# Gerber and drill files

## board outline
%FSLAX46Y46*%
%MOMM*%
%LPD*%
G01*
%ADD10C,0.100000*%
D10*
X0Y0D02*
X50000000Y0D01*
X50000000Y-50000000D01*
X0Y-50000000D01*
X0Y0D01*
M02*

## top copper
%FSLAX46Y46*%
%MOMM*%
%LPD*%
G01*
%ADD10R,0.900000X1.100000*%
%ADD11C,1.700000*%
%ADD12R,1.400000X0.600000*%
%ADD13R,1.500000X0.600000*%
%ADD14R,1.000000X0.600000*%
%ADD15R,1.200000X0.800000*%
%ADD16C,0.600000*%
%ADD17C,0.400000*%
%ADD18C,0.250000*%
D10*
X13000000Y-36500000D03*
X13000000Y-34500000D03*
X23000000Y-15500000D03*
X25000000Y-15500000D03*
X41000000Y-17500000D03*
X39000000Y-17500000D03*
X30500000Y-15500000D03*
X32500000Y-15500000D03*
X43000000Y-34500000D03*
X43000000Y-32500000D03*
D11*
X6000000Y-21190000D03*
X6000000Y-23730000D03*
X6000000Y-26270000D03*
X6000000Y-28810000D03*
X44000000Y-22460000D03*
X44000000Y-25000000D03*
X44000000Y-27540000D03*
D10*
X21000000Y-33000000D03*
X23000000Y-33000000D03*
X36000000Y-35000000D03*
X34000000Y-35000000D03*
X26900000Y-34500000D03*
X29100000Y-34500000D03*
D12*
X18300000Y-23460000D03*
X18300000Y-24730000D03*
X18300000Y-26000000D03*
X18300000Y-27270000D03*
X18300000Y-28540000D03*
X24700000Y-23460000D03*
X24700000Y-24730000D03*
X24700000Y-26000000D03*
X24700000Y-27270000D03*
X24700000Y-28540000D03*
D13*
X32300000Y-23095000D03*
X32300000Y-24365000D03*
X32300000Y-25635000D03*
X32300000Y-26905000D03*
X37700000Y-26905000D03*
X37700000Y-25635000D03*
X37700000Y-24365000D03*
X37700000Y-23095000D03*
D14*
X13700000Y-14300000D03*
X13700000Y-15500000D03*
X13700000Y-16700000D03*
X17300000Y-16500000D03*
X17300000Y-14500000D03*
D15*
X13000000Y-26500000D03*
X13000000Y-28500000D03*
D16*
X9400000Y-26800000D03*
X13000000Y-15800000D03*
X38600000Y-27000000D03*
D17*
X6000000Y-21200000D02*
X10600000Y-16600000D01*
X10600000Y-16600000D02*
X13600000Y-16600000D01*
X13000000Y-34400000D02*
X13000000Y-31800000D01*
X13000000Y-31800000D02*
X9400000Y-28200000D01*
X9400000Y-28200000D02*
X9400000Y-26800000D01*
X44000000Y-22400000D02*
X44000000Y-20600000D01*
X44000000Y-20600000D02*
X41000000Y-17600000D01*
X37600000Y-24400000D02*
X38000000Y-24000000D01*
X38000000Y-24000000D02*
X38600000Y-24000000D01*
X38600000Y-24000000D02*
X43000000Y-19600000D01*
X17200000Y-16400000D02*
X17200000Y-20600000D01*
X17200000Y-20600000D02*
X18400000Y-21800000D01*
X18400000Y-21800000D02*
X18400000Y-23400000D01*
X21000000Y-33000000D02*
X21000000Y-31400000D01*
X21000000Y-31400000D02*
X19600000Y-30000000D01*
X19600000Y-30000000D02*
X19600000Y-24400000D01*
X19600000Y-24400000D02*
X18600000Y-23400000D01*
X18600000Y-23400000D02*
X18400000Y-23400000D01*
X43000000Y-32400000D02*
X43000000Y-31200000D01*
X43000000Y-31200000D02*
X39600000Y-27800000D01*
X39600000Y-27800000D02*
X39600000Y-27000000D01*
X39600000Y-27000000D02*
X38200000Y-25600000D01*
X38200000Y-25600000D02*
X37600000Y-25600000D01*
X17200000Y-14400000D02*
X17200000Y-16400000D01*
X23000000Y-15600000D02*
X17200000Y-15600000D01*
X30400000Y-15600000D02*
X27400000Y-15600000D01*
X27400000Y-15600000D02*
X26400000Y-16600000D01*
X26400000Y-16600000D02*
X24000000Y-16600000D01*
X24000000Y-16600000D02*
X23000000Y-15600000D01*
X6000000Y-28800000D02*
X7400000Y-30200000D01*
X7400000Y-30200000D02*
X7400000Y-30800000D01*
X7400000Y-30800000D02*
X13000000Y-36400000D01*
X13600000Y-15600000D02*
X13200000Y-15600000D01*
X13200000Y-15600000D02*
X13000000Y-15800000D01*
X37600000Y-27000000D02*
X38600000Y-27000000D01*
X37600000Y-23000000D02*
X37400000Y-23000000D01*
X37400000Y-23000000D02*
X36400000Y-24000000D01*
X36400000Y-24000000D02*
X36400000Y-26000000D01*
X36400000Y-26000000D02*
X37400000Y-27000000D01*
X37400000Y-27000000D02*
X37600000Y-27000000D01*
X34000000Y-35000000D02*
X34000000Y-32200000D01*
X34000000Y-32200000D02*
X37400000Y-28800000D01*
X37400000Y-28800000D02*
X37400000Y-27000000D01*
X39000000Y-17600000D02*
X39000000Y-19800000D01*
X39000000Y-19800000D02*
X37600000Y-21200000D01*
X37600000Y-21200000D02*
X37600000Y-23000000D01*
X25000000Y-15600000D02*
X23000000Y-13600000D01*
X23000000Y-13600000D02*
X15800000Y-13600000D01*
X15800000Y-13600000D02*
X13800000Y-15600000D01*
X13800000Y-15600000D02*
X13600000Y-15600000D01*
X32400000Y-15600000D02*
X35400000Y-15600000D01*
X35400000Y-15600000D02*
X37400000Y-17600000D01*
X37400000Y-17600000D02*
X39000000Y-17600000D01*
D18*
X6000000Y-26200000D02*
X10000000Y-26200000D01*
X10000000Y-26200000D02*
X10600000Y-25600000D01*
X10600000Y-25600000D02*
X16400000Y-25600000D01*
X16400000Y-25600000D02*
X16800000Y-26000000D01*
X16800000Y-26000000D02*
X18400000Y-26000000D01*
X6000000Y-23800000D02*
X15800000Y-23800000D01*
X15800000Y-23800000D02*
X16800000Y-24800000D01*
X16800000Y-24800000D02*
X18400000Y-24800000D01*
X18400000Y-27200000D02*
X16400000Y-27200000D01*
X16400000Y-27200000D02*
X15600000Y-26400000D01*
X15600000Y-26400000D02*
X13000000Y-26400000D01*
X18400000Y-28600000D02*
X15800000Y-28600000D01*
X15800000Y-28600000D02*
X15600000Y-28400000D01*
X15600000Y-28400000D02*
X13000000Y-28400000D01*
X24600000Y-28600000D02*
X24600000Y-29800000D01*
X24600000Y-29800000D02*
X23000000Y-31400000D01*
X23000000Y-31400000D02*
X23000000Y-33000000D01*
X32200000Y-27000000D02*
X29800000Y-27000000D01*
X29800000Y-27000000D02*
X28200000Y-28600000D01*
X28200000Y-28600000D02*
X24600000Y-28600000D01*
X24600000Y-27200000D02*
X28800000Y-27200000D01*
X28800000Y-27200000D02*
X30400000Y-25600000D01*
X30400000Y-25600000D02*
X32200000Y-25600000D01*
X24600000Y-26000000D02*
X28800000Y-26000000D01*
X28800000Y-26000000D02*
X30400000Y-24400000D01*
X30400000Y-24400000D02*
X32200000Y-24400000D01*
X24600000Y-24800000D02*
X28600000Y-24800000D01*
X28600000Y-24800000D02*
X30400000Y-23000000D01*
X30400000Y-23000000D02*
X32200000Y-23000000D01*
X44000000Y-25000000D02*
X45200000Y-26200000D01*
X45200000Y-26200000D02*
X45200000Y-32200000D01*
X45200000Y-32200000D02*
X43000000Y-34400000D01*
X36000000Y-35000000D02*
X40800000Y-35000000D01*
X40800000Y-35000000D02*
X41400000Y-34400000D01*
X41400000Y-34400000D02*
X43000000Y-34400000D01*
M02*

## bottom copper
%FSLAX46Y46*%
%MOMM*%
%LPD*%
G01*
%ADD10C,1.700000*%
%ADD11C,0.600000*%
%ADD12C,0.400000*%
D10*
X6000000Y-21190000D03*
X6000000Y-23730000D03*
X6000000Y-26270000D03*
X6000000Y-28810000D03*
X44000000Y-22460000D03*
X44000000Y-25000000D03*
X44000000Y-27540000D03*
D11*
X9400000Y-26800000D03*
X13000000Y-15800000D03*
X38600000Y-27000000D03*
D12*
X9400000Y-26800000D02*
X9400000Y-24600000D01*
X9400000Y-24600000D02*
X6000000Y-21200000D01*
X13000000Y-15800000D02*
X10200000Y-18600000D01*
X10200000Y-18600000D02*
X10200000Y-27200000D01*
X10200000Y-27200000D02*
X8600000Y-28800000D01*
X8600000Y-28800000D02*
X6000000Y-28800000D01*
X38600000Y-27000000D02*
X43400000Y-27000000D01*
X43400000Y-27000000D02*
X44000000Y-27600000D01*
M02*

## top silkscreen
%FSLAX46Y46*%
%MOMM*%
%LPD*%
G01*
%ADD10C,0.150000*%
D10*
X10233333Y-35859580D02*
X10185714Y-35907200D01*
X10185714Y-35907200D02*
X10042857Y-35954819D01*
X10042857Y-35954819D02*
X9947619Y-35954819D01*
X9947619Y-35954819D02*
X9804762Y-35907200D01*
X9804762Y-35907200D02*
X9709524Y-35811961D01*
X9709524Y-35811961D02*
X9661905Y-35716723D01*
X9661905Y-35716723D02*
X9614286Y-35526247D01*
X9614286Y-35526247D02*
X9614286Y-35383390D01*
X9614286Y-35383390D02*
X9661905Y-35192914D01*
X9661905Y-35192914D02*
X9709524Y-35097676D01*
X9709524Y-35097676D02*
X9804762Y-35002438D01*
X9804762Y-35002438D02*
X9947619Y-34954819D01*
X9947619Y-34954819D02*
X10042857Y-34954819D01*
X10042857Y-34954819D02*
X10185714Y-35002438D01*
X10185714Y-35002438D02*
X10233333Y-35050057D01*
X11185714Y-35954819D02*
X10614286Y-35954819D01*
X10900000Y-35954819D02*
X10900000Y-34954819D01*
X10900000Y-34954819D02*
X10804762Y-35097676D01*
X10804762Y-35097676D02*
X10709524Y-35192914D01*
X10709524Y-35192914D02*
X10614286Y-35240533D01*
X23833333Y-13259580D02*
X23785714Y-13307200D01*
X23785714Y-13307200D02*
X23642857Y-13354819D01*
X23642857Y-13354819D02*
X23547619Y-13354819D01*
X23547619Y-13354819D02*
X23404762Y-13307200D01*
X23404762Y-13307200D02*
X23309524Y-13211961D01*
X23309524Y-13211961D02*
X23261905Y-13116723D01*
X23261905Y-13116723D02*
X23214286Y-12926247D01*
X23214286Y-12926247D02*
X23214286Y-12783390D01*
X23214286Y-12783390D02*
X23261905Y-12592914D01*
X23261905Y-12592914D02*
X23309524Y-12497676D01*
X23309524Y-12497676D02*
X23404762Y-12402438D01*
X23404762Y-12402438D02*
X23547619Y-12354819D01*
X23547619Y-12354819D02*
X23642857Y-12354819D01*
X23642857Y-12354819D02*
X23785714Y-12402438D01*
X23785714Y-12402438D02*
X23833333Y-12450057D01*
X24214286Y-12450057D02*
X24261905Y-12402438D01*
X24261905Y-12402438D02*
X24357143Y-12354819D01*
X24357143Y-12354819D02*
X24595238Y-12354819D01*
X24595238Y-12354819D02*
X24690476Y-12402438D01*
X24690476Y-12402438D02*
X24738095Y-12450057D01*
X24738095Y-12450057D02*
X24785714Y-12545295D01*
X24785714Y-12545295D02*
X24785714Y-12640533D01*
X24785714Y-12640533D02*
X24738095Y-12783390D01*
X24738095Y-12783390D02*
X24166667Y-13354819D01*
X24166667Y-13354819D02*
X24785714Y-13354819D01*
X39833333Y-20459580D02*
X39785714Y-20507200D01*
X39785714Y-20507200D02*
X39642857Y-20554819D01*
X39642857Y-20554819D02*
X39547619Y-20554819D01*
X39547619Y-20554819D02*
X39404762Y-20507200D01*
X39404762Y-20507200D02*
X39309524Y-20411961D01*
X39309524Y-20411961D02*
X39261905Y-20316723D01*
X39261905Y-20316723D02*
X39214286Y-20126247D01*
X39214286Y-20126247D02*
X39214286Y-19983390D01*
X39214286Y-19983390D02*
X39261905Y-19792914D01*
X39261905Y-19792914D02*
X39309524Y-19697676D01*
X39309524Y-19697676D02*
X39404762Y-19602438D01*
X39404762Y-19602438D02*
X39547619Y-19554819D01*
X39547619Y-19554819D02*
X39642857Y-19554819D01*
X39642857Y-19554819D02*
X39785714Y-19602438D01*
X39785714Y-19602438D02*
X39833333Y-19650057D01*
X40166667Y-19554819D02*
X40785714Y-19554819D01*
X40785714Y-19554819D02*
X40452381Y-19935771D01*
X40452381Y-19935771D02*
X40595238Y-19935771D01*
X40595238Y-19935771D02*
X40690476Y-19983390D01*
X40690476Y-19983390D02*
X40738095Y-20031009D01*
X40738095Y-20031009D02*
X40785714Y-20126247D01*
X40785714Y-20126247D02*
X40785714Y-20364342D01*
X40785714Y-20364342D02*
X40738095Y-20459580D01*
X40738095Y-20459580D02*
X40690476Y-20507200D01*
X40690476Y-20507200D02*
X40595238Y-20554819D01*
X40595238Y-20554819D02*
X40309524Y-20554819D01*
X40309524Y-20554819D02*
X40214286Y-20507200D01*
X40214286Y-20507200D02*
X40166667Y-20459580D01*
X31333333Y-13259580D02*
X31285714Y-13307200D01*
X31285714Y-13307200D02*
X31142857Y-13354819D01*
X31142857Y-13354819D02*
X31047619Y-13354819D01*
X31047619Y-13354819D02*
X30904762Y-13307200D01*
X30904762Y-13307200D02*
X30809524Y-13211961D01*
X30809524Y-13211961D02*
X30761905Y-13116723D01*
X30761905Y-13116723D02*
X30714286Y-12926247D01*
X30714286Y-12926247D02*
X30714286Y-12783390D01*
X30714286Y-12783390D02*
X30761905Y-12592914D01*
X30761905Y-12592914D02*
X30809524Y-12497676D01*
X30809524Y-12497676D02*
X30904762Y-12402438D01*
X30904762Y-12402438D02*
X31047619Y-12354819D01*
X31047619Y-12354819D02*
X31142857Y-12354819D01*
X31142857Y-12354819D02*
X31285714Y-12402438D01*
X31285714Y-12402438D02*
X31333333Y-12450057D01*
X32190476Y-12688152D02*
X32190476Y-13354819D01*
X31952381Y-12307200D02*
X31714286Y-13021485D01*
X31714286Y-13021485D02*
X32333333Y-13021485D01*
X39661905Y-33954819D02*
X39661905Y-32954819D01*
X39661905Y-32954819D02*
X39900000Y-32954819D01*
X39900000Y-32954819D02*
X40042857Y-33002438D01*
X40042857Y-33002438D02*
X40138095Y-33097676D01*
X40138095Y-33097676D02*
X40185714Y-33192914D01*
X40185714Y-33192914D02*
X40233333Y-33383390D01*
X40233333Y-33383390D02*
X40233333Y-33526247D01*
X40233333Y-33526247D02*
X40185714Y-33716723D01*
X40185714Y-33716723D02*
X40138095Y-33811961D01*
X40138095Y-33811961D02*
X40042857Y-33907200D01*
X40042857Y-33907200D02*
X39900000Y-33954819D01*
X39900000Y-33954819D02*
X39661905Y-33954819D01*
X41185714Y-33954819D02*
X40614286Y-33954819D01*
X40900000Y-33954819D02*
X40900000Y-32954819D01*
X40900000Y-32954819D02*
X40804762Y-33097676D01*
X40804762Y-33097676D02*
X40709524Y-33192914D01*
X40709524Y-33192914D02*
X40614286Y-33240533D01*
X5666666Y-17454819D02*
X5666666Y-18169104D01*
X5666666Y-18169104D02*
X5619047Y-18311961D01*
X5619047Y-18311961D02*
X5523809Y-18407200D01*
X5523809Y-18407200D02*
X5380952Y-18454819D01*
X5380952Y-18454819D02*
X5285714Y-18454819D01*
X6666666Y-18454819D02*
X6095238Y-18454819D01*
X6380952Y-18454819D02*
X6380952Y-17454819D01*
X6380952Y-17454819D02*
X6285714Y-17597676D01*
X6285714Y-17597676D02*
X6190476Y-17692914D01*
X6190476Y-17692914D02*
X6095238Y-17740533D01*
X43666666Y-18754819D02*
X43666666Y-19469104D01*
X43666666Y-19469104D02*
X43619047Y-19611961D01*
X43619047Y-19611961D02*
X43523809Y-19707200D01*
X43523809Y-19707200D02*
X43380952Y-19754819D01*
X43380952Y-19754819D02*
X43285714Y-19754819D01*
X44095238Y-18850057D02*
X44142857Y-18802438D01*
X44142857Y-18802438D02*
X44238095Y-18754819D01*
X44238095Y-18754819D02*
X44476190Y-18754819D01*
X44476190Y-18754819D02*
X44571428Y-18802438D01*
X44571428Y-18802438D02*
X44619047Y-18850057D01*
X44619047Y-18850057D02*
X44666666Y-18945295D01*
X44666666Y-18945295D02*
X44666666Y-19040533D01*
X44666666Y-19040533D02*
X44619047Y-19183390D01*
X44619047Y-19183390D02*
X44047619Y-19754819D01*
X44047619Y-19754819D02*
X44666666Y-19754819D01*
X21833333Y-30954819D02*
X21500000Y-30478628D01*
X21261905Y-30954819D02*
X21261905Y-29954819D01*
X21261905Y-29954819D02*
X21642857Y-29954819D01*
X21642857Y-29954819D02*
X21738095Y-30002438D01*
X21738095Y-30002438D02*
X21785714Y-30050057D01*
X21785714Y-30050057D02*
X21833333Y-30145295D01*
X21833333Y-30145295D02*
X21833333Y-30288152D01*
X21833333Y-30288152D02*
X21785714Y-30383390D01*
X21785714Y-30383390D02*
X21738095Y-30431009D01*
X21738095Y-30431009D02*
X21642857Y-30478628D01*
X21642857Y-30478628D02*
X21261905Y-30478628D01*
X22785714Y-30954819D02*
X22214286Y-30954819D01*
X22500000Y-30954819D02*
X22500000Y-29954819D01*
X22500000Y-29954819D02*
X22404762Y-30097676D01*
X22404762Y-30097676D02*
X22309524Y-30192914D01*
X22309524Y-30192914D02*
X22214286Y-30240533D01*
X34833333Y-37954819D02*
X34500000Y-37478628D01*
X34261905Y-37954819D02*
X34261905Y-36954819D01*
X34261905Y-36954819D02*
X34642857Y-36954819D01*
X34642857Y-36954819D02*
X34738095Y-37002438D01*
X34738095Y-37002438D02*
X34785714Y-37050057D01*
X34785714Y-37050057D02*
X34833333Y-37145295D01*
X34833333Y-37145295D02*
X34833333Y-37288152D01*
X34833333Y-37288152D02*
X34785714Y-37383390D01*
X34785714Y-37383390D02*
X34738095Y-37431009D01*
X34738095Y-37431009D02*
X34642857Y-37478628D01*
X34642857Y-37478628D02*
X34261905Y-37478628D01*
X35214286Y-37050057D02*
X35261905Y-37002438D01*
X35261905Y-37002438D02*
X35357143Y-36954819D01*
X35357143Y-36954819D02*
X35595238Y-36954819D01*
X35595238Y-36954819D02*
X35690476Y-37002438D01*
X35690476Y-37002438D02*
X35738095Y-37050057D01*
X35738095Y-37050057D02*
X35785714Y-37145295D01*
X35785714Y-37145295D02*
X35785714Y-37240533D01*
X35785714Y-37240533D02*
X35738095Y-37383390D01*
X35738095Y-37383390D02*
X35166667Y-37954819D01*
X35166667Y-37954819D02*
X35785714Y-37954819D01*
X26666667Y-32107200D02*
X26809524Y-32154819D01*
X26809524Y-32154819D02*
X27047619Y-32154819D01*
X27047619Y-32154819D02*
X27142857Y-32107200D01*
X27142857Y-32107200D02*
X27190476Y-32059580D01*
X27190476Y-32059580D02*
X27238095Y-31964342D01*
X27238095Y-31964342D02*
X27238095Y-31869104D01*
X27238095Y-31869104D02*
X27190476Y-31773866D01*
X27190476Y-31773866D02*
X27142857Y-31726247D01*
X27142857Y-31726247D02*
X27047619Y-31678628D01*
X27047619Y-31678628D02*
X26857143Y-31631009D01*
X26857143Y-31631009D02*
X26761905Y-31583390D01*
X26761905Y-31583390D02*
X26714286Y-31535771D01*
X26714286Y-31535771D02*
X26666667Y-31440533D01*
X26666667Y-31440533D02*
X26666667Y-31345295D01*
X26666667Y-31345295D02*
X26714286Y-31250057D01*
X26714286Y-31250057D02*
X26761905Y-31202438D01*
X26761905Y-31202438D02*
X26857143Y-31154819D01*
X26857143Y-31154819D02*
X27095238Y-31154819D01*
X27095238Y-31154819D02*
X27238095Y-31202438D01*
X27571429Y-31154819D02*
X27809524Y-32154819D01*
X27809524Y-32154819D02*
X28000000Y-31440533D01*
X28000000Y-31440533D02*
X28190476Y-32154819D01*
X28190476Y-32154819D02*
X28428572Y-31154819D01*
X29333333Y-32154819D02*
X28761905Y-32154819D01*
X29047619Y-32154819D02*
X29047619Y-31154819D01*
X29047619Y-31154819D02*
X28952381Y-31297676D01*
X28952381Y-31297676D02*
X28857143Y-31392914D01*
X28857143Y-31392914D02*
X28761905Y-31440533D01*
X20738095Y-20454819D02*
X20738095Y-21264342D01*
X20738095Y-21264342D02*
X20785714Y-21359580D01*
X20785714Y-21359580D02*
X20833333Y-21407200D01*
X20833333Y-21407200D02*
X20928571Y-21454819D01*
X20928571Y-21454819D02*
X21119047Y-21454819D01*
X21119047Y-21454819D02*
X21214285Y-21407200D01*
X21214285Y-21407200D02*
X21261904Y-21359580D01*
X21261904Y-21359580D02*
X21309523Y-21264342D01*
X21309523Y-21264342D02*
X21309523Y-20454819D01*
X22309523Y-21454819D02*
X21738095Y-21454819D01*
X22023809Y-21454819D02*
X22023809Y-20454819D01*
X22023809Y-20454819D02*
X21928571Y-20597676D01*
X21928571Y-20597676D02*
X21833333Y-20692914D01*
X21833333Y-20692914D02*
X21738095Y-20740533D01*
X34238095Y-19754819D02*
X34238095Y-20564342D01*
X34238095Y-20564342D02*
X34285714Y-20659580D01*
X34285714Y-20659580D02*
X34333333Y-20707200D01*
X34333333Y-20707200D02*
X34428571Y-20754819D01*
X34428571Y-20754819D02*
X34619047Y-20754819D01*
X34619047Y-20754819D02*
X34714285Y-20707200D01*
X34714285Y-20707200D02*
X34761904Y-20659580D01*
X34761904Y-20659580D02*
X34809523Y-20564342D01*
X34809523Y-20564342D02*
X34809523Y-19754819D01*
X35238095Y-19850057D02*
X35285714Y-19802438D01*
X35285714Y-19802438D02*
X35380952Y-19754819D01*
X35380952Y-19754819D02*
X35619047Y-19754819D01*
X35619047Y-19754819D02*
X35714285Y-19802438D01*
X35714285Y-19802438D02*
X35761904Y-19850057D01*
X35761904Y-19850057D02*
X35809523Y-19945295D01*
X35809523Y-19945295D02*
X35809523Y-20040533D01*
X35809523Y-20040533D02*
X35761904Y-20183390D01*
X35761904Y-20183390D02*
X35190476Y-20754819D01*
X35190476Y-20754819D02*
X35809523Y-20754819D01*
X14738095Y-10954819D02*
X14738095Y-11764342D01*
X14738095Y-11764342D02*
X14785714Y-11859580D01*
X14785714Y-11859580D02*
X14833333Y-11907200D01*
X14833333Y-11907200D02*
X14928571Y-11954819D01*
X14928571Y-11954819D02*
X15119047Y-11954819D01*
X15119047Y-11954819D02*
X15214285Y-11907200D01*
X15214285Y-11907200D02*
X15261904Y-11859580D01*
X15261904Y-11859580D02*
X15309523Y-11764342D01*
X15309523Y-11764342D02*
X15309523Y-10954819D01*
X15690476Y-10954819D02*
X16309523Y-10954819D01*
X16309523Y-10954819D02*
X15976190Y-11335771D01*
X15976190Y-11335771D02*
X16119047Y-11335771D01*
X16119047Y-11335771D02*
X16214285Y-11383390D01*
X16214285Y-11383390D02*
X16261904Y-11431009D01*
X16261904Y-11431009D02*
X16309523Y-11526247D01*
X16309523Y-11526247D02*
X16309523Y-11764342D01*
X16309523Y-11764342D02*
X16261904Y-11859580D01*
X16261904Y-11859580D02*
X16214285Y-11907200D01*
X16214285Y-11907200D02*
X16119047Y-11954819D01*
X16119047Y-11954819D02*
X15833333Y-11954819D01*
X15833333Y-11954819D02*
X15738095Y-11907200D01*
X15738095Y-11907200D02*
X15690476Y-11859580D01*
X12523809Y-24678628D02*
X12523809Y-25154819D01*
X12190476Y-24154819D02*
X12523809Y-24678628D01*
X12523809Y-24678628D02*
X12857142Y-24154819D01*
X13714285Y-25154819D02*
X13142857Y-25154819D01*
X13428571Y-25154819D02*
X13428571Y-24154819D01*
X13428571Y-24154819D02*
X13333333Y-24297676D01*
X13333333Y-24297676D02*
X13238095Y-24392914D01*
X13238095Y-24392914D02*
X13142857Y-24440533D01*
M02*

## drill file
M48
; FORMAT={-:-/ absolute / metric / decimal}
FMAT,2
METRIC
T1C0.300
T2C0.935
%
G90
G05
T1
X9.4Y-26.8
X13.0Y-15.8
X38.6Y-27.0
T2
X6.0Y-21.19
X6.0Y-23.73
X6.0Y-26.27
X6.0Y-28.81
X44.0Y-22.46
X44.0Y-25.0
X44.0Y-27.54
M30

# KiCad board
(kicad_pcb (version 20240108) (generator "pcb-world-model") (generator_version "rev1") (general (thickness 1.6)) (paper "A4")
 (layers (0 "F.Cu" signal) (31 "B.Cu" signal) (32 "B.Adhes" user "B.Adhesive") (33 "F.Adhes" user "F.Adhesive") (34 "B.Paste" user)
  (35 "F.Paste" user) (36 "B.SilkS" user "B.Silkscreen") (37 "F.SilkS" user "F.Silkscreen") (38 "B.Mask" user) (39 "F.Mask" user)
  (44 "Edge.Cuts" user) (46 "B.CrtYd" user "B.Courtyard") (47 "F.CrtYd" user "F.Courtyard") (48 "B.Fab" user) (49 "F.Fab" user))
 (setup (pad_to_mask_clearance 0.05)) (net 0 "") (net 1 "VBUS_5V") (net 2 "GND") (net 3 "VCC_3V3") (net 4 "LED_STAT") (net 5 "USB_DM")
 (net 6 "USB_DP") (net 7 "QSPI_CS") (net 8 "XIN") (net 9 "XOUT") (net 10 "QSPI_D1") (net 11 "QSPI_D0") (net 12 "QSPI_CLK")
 (gr_rect (start 0.0 0.0) (end 50.0000 50.0000) (stroke (width 0.1) (type default)) (fill none) (layer "Edge.Cuts"))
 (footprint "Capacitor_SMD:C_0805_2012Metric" (layer "F.Cu") (at 13.0000 35.5000 90)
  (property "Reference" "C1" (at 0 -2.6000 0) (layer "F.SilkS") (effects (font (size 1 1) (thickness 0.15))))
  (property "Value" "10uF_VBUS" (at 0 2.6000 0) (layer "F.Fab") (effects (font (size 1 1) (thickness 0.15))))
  (pad "1" smd rect (at -1.0000 0.0000) (size 0.9000 1.1000) (layers "F.Cu" "F.Paste" "F.Mask") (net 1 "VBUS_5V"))
  (pad "2" smd rect (at 1.0000 0.0000) (size 0.9000 1.1000) (layers "F.Cu" "F.Paste" "F.Mask") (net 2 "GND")))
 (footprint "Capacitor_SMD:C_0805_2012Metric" (layer "F.Cu") (at 24.0000 15.5000 0)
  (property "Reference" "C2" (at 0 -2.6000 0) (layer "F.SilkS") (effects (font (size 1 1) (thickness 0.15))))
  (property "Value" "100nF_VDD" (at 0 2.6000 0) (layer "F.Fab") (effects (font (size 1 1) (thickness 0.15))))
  (pad "1" smd rect (at -1.0000 0.0000) (size 0.9000 1.1000) (layers "F.Cu" "F.Paste" "F.Mask") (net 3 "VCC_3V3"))
  (pad "2" smd rect (at 1.0000 0.0000) (size 0.9000 1.1000) (layers "F.Cu" "F.Paste" "F.Mask") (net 2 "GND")))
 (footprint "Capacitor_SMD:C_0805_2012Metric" (layer "F.Cu") (at 40.0000 17.5000 180)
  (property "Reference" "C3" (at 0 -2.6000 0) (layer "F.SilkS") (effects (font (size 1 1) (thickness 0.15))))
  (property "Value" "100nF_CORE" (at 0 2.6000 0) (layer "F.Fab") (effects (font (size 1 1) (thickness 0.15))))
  (pad "1" smd rect (at -1.0000 0.0000) (size 0.9000 1.1000) (layers "F.Cu" "F.Paste" "F.Mask") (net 3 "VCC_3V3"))
  (pad "2" smd rect (at 1.0000 0.0000) (size 0.9000 1.1000) (layers "F.Cu" "F.Paste" "F.Mask") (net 2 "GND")))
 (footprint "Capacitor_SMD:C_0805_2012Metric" (layer "F.Cu") (at 31.5000 15.5000 0)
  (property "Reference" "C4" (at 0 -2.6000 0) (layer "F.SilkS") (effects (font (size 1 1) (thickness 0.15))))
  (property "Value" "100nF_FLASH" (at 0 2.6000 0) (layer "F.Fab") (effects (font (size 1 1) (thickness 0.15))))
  (pad "1" smd rect (at -1.0000 0.0000) (size 0.9000 1.1000) (layers "F.Cu" "F.Paste" "F.Mask") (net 3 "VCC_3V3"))
  (pad "2" smd rect (at 1.0000 0.0000) (size 0.9000 1.1000) (layers "F.Cu" "F.Paste" "F.Mask") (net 2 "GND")))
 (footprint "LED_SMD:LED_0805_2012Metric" (layer "F.Cu") (at 43.0000 33.5000 90)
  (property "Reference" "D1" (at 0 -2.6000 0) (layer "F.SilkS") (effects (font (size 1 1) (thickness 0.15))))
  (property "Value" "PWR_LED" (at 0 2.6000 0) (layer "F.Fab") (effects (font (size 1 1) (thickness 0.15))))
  (pad "1" smd rect (at -1.0000 0.0000) (size 0.9000 1.1000) (layers "F.Cu" "F.Paste" "F.Mask") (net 3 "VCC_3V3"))
  (pad "2" smd rect (at 1.0000 0.0000) (size 0.9000 1.1000) (layers "F.Cu" "F.Paste" "F.Mask") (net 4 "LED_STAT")))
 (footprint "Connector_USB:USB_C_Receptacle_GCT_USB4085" (layer "F.Cu") (at 6.0000 25.0000 0) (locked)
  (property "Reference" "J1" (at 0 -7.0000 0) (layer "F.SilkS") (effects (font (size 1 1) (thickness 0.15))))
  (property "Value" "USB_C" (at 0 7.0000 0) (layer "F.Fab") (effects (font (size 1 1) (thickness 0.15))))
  (pad "1" thru_hole circle (at 0.0000 -3.8100) (size 1.7000 1.7000) (drill 0.9350) (layers "*.Cu" "*.Mask") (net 1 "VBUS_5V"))
  (pad "2" thru_hole circle (at 0.0000 -1.2700) (size 1.7000 1.7000) (drill 0.9350) (layers "*.Cu" "*.Mask") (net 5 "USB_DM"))
  (pad "3" thru_hole circle (at 0.0000 1.2700) (size 1.7000 1.7000) (drill 0.9350) (layers "*.Cu" "*.Mask") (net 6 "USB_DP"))
  (pad "4" thru_hole circle (at 0.0000 3.8100) (size 1.7000 1.7000) (drill 0.9350) (layers "*.Cu" "*.Mask") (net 2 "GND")))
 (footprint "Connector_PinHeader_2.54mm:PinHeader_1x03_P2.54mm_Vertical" (layer "F.Cu") (at 44.0000 25.0000 0) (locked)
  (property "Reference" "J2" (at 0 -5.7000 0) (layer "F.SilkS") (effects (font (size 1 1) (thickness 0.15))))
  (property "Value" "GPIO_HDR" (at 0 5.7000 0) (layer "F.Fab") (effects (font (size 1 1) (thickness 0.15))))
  (pad "1" thru_hole circle (at 0.0000 -2.5400) (size 1.7000 1.7000) (drill 0.9350) (layers "*.Cu" "*.Mask") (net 3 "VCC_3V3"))
  (pad "2" thru_hole circle (at 0.0000 0.0000) (size 1.7000 1.7000) (drill 0.9350) (layers "*.Cu" "*.Mask") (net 4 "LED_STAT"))
  (pad "3" thru_hole circle (at 0.0000 2.5400) (size 1.7000 1.7000) (drill 0.9350) (layers "*.Cu" "*.Mask") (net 2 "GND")))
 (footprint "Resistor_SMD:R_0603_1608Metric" (layer "F.Cu") (at 22.0000 33.0000 0)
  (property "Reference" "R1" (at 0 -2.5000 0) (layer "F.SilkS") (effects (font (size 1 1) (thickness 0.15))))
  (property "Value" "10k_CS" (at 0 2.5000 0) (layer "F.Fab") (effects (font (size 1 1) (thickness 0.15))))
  (pad "1" smd rect (at -1.0000 0.0000) (size 0.9000 1.1000) (layers "F.Cu" "F.Paste" "F.Mask") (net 3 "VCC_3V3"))
  (pad "2" smd rect (at 1.0000 0.0000) (size 0.9000 1.1000) (layers "F.Cu" "F.Paste" "F.Mask") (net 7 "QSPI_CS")))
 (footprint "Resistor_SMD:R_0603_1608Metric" (layer "F.Cu") (at 35.0000 35.0000 180)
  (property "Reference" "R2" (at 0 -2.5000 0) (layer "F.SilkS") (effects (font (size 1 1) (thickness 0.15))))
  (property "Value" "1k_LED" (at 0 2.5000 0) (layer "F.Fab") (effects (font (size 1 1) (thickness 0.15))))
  (pad "1" smd rect (at -1.0000 0.0000) (size 0.9000 1.1000) (layers "F.Cu" "F.Paste" "F.Mask") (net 4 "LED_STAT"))
  (pad "2" smd rect (at 1.0000 0.0000) (size 0.9000 1.1000) (layers "F.Cu" "F.Paste" "F.Mask") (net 2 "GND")))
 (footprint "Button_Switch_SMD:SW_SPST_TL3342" (layer "F.Cu") (at 28.0000 34.5000 0)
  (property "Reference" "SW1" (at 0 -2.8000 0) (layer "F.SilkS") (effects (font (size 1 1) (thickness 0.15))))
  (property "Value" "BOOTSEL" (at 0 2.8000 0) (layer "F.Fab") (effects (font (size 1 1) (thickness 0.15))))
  (pad "1" smd rect (at -1.1000 0.0000) (size 0.9000 1.1000) (layers "F.Cu" "F.Paste" "F.Mask") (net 7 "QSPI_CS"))
  (pad "2" smd rect (at 1.1000 0.0000) (size 0.9000 1.1000) (layers "F.Cu" "F.Paste" "F.Mask") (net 2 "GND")))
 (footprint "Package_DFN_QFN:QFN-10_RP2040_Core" (layer "F.Cu") (at 21.5000 26.0000 0)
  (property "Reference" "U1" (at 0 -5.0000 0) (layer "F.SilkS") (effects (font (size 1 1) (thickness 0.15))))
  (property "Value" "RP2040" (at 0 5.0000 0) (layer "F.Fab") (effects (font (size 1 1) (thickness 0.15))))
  (pad "1" smd rect (at -3.2000 -2.5400) (size 1.4000 0.6000) (layers "F.Cu" "F.Paste" "F.Mask") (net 3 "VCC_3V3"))
  (pad "2" smd rect (at -3.2000 -1.2700) (size 1.4000 0.6000) (layers "F.Cu" "F.Paste" "F.Mask") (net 5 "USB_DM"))
  (pad "3" smd rect (at -3.2000 0.0000) (size 1.4000 0.6000) (layers "F.Cu" "F.Paste" "F.Mask") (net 6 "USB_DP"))
  (pad "4" smd rect (at -3.2000 1.2700) (size 1.4000 0.6000) (layers "F.Cu" "F.Paste" "F.Mask") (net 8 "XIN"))
  (pad "5" smd rect (at -3.2000 2.5400) (size 1.4000 0.6000) (layers "F.Cu" "F.Paste" "F.Mask") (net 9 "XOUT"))
  (pad "6" smd rect (at 3.2000 -2.5400) (size 1.4000 0.6000) (layers "F.Cu" "F.Paste" "F.Mask") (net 4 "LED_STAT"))
  (pad "7" smd rect (at 3.2000 -1.2700) (size 1.4000 0.6000) (layers "F.Cu" "F.Paste" "F.Mask") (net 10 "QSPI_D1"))
  (pad "8" smd rect (at 3.2000 0.0000) (size 1.4000 0.6000) (layers "F.Cu" "F.Paste" "F.Mask") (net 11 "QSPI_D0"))
  (pad "9" smd rect (at 3.2000 1.2700) (size 1.4000 0.6000) (layers "F.Cu" "F.Paste" "F.Mask") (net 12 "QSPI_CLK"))
  (pad "10" smd rect (at 3.2000 2.5400) (size 1.4000 0.6000) (layers "F.Cu" "F.Paste" "F.Mask") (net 7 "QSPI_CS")))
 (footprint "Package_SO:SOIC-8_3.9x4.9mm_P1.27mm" (layer "F.Cu") (at 35.0000 25.0000 0)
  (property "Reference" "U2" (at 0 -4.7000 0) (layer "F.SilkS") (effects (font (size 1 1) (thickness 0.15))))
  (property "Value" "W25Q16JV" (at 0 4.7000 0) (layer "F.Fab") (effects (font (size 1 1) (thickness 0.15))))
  (pad "1" smd rect (at -2.7000 -1.9050) (size 1.5000 0.6000) (layers "F.Cu" "F.Paste" "F.Mask") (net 10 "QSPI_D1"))
  (pad "2" smd rect (at -2.7000 -0.6350) (size 1.5000 0.6000) (layers "F.Cu" "F.Paste" "F.Mask") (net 11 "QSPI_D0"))
  (pad "3" smd rect (at -2.7000 0.6350) (size 1.5000 0.6000) (layers "F.Cu" "F.Paste" "F.Mask") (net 12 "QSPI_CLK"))
  (pad "4" smd rect (at -2.7000 1.9050) (size 1.5000 0.6000) (layers "F.Cu" "F.Paste" "F.Mask") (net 7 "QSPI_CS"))
  (pad "5" smd rect (at 2.7000 1.9050) (size 1.5000 0.6000) (layers "F.Cu" "F.Paste" "F.Mask") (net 2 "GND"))
  (pad "6" smd rect (at 2.7000 0.6350) (size 1.5000 0.6000) (layers "F.Cu" "F.Paste" "F.Mask") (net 3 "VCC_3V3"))
  (pad "7" smd rect (at 2.7000 -0.6350) (size 1.5000 0.6000) (layers "F.Cu" "F.Paste" "F.Mask") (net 3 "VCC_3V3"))
  (pad "8" smd rect (at 2.7000 -1.9050) (size 1.5000 0.6000) (layers "F.Cu" "F.Paste" "F.Mask") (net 2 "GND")))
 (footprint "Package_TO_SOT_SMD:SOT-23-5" (layer "F.Cu") (at 15.5000 15.5000 0)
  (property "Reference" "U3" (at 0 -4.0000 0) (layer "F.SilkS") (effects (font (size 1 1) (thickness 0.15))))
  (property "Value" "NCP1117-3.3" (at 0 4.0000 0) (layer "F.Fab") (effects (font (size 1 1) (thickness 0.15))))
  (pad "1" smd rect (at -1.8000 -1.2000) (size 1.0000 0.6000) (layers "F.Cu" "F.Paste" "F.Mask") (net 1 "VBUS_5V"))
  (pad "2" smd rect (at -1.8000 0.0000) (size 1.0000 0.6000) (layers "F.Cu" "F.Paste" "F.Mask") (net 2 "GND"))
  (pad "3" smd rect (at -1.8000 1.2000) (size 1.0000 0.6000) (layers "F.Cu" "F.Paste" "F.Mask") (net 1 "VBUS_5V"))
  (pad "4" smd rect (at 1.8000 1.0000) (size 1.0000 0.6000) (layers "F.Cu" "F.Paste" "F.Mask") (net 3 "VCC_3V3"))
  (pad "5" smd rect (at 1.8000 -1.0000) (size 1.0000 0.6000) (layers "F.Cu" "F.Paste" "F.Mask") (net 3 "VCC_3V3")))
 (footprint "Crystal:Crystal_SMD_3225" (layer "F.Cu") (at 13.0000 27.5000 0)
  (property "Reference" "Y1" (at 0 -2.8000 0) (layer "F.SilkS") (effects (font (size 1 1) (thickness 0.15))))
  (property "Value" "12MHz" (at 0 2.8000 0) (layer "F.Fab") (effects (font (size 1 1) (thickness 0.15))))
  (pad "1" smd rect (at 0.0000 -1.0000) (size 1.2000 0.8000) (layers "F.Cu" "F.Paste" "F.Mask") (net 8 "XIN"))
  (pad "2" smd rect (at 0.0000 1.0000) (size 1.2000 0.8000) (layers "F.Cu" "F.Paste" "F.Mask") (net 9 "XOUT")))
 (segment (start 6.0000 21.2000) (end 10.6000 16.6000) (width 0.4000) (layer "F.Cu") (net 1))
 (segment (start 10.6000 16.6000) (end 13.6000 16.6000) (width 0.4000) (layer "F.Cu") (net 1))
 (segment (start 13.0000 34.4000) (end 13.0000 31.8000) (width 0.4000) (layer "F.Cu") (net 1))
 (segment (start 13.0000 31.8000) (end 9.4000 28.2000) (width 0.4000) (layer "F.Cu") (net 1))
 (segment (start 9.4000 28.2000) (end 9.4000 26.8000) (width 0.4000) (layer "F.Cu") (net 1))
 (segment (start 9.4000 26.8000) (end 9.4000 24.6000) (width 0.4000) (layer "B.Cu") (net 1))
 (segment (start 9.4000 24.6000) (end 6.0000 21.2000) (width 0.4000) (layer "B.Cu") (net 1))
 (segment (start 44.0000 22.4000) (end 44.0000 20.6000) (width 0.4000) (layer "F.Cu") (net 3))
 (segment (start 44.0000 20.6000) (end 41.0000 17.6000) (width 0.4000) (layer "F.Cu") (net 3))
 (segment (start 37.6000 24.4000) (end 38.0000 24.0000) (width 0.4000) (layer "F.Cu") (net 3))
 (segment (start 38.0000 24.0000) (end 38.6000 24.0000) (width 0.4000) (layer "F.Cu") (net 3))
 (segment (start 38.6000 24.0000) (end 43.0000 19.6000) (width 0.4000) (layer "F.Cu") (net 3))
 (segment (start 17.2000 16.4000) (end 17.2000 20.6000) (width 0.4000) (layer "F.Cu") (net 3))
 (segment (start 17.2000 20.6000) (end 18.4000 21.8000) (width 0.4000) (layer "F.Cu") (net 3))
 (segment (start 18.4000 21.8000) (end 18.4000 23.4000) (width 0.4000) (layer "F.Cu") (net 3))
 (segment (start 21.0000 33.0000) (end 21.0000 31.4000) (width 0.4000) (layer "F.Cu") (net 3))
 (segment (start 21.0000 31.4000) (end 19.6000 30.0000) (width 0.4000) (layer "F.Cu") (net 3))
 (segment (start 19.6000 30.0000) (end 19.6000 24.4000) (width 0.4000) (layer "F.Cu") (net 3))
 (segment (start 19.6000 24.4000) (end 18.6000 23.4000) (width 0.4000) (layer "F.Cu") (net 3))
 (segment (start 18.6000 23.4000) (end 18.4000 23.4000) (width 0.4000) (layer "F.Cu") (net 3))
 (segment (start 43.0000 32.4000) (end 43.0000 31.2000) (width 0.4000) (layer "F.Cu") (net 3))
 (segment (start 43.0000 31.2000) (end 39.6000 27.8000) (width 0.4000) (layer "F.Cu") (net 3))
 (segment (start 39.6000 27.8000) (end 39.6000 27.0000) (width 0.4000) (layer "F.Cu") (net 3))
 (segment (start 39.6000 27.0000) (end 38.2000 25.6000) (width 0.4000) (layer "F.Cu") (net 3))
 (segment (start 38.2000 25.6000) (end 37.6000 25.6000) (width 0.4000) (layer "F.Cu") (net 3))
 (segment (start 17.2000 14.4000) (end 17.2000 16.4000) (width 0.4000) (layer "F.Cu") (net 3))
 (segment (start 23.0000 15.6000) (end 17.2000 15.6000) (width 0.4000) (layer "F.Cu") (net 3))
 (segment (start 30.4000 15.6000) (end 27.4000 15.6000) (width 0.4000) (layer "F.Cu") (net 3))
 (segment (start 27.4000 15.6000) (end 26.4000 16.6000) (width 0.4000) (layer "F.Cu") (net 3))
 (segment (start 26.4000 16.6000) (end 24.0000 16.6000) (width 0.4000) (layer "F.Cu") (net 3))
 (segment (start 24.0000 16.6000) (end 23.0000 15.6000) (width 0.4000) (layer "F.Cu") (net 3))
 (segment (start 6.0000 28.8000) (end 7.4000 30.2000) (width 0.4000) (layer "F.Cu") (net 2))
 (segment (start 7.4000 30.2000) (end 7.4000 30.8000) (width 0.4000) (layer "F.Cu") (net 2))
 (segment (start 7.4000 30.8000) (end 13.0000 36.4000) (width 0.4000) (layer "F.Cu") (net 2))
 (segment (start 13.6000 15.6000) (end 13.2000 15.6000) (width 0.4000) (layer "F.Cu") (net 2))
 (segment (start 13.2000 15.6000) (end 13.0000 15.8000) (width 0.4000) (layer "F.Cu") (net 2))
 (segment (start 13.0000 15.8000) (end 10.2000 18.6000) (width 0.4000) (layer "B.Cu") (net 2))
 (segment (start 10.2000 18.6000) (end 10.2000 27.2000) (width 0.4000) (layer "B.Cu") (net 2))
 (segment (start 10.2000 27.2000) (end 8.6000 28.8000) (width 0.4000) (layer "B.Cu") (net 2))
 (segment (start 8.6000 28.8000) (end 6.0000 28.8000) (width 0.4000) (layer "B.Cu") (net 2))
 (segment (start 37.6000 27.0000) (end 38.6000 27.0000) (width 0.4000) (layer "F.Cu") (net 2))
 (segment (start 38.6000 27.0000) (end 43.4000 27.0000) (width 0.4000) (layer "B.Cu") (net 2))
 (segment (start 43.4000 27.0000) (end 44.0000 27.6000) (width 0.4000) (layer "B.Cu") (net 2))
 (segment (start 37.6000 23.0000) (end 37.4000 23.0000) (width 0.4000) (layer "F.Cu") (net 2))
 (segment (start 37.4000 23.0000) (end 36.4000 24.0000) (width 0.4000) (layer "F.Cu") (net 2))
 (segment (start 36.4000 24.0000) (end 36.4000 26.0000) (width 0.4000) (layer "F.Cu") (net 2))
 (segment (start 36.4000 26.0000) (end 37.4000 27.0000) (width 0.4000) (layer "F.Cu") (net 2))
 (segment (start 37.4000 27.0000) (end 37.6000 27.0000) (width 0.4000) (layer "F.Cu") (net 2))
 (segment (start 34.0000 35.0000) (end 34.0000 32.2000) (width 0.4000) (layer "F.Cu") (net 2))
 (segment (start 34.0000 32.2000) (end 37.4000 28.8000) (width 0.4000) (layer "F.Cu") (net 2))
 (segment (start 37.4000 28.8000) (end 37.4000 27.0000) (width 0.4000) (layer "F.Cu") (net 2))
 (segment (start 39.0000 17.6000) (end 39.0000 19.8000) (width 0.4000) (layer "F.Cu") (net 2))
 (segment (start 39.0000 19.8000) (end 37.6000 21.2000) (width 0.4000) (layer "F.Cu") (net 2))
 (segment (start 37.6000 21.2000) (end 37.6000 23.0000) (width 0.4000) (layer "F.Cu") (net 2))
 (segment (start 25.0000 15.6000) (end 23.0000 13.6000) (width 0.4000) (layer "F.Cu") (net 2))
 (segment (start 23.0000 13.6000) (end 15.8000 13.6000) (width 0.4000) (layer "F.Cu") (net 2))
 (segment (start 15.8000 13.6000) (end 13.8000 15.6000) (width 0.4000) (layer "F.Cu") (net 2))
 (segment (start 13.8000 15.6000) (end 13.6000 15.6000) (width 0.4000) (layer "F.Cu") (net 2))
 (segment (start 32.4000 15.6000) (end 35.4000 15.6000) (width 0.4000) (layer "F.Cu") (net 2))
 (segment (start 35.4000 15.6000) (end 37.4000 17.6000) (width 0.4000) (layer "F.Cu") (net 2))
 (segment (start 37.4000 17.6000) (end 39.0000 17.6000) (width 0.4000) (layer "F.Cu") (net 2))
 (segment (start 6.0000 26.2000) (end 10.0000 26.2000) (width 0.2500) (layer "F.Cu") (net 6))
 (segment (start 10.0000 26.2000) (end 10.6000 25.6000) (width 0.2500) (layer "F.Cu") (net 6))
 (segment (start 10.6000 25.6000) (end 16.4000 25.6000) (width 0.2500) (layer "F.Cu") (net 6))
 (segment (start 16.4000 25.6000) (end 16.8000 26.0000) (width 0.2500) (layer "F.Cu") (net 6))
 (segment (start 16.8000 26.0000) (end 18.4000 26.0000) (width 0.2500) (layer "F.Cu") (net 6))
 (segment (start 6.0000 23.8000) (end 15.8000 23.8000) (width 0.2500) (layer "F.Cu") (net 5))
 (segment (start 15.8000 23.8000) (end 16.8000 24.8000) (width 0.2500) (layer "F.Cu") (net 5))
 (segment (start 16.8000 24.8000) (end 18.4000 24.8000) (width 0.2500) (layer "F.Cu") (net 5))
 (segment (start 18.4000 27.2000) (end 16.4000 27.2000) (width 0.2500) (layer "F.Cu") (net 8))
 (segment (start 16.4000 27.2000) (end 15.6000 26.4000) (width 0.2500) (layer "F.Cu") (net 8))
 (segment (start 15.6000 26.4000) (end 13.0000 26.4000) (width 0.2500) (layer "F.Cu") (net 8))
 (segment (start 18.4000 28.6000) (end 15.8000 28.6000) (width 0.2500) (layer "F.Cu") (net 9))
 (segment (start 15.8000 28.6000) (end 15.6000 28.4000) (width 0.2500) (layer "F.Cu") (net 9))
 (segment (start 15.6000 28.4000) (end 13.0000 28.4000) (width 0.2500) (layer "F.Cu") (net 9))
 (segment (start 24.6000 28.6000) (end 24.6000 29.8000) (width 0.2500) (layer "F.Cu") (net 7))
 (segment (start 24.6000 29.8000) (end 23.0000 31.4000) (width 0.2500) (layer "F.Cu") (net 7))
 (segment (start 23.0000 31.4000) (end 23.0000 33.0000) (width 0.2500) (layer "F.Cu") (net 7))
 (segment (start 32.2000 27.0000) (end 29.8000 27.0000) (width 0.2500) (layer "F.Cu") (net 7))
 (segment (start 29.8000 27.0000) (end 28.2000 28.6000) (width 0.2500) (layer "F.Cu") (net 7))
 (segment (start 28.2000 28.6000) (end 24.6000 28.6000) (width 0.2500) (layer "F.Cu") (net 7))
 (segment (start 24.6000 27.2000) (end 28.8000 27.2000) (width 0.2500) (layer "F.Cu") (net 12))
 (segment (start 28.8000 27.2000) (end 30.4000 25.6000) (width 0.2500) (layer "F.Cu") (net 12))
 (segment (start 30.4000 25.6000) (end 32.2000 25.6000) (width 0.2500) (layer "F.Cu") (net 12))
 (segment (start 24.6000 26.0000) (end 28.8000 26.0000) (width 0.2500) (layer "F.Cu") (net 11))
 (segment (start 28.8000 26.0000) (end 30.4000 24.4000) (width 0.2500) (layer "F.Cu") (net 11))
 (segment (start 30.4000 24.4000) (end 32.2000 24.4000) (width 0.2500) (layer "F.Cu") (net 11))
 (segment (start 24.6000 24.8000) (end 28.6000 24.8000) (width 0.2500) (layer "F.Cu") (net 10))
 (segment (start 28.6000 24.8000) (end 30.4000 23.0000) (width 0.2500) (layer "F.Cu") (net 10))
 (segment (start 30.4000 23.0000) (end 32.2000 23.0000) (width 0.2500) (layer "F.Cu") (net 10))
 (segment (start 44.0000 25.0000) (end 45.2000 26.2000) (width 0.2500) (layer "F.Cu") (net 4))
 (segment (start 45.2000 26.2000) (end 45.2000 32.2000) (width 0.2500) (layer "F.Cu") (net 4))
 (segment (start 45.2000 32.2000) (end 43.0000 34.4000) (width 0.2500) (layer "F.Cu") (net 4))
 (segment (start 36.0000 35.0000) (end 40.8000 35.0000) (width 0.2500) (layer "F.Cu") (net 4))
 (segment (start 40.8000 35.0000) (end 41.4000 34.4000) (width 0.2500) (layer "F.Cu") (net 4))
 (segment (start 41.4000 34.4000) (end 43.0000 34.4000) (width 0.2500) (layer "F.Cu") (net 4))
 (via (at 9.4000 26.8000) (size 0.6000) (drill 0.3000) (layers "F.Cu" "B.Cu") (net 1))
 (via (at 13.0000 15.8000) (size 0.6000) (drill 0.3000) (layers "F.Cu" "B.Cu") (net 2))
 (via (at 38.6000 27.0000) (size 0.6000) (drill 0.3000) (layers "F.Cu" "B.Cu") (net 2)))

